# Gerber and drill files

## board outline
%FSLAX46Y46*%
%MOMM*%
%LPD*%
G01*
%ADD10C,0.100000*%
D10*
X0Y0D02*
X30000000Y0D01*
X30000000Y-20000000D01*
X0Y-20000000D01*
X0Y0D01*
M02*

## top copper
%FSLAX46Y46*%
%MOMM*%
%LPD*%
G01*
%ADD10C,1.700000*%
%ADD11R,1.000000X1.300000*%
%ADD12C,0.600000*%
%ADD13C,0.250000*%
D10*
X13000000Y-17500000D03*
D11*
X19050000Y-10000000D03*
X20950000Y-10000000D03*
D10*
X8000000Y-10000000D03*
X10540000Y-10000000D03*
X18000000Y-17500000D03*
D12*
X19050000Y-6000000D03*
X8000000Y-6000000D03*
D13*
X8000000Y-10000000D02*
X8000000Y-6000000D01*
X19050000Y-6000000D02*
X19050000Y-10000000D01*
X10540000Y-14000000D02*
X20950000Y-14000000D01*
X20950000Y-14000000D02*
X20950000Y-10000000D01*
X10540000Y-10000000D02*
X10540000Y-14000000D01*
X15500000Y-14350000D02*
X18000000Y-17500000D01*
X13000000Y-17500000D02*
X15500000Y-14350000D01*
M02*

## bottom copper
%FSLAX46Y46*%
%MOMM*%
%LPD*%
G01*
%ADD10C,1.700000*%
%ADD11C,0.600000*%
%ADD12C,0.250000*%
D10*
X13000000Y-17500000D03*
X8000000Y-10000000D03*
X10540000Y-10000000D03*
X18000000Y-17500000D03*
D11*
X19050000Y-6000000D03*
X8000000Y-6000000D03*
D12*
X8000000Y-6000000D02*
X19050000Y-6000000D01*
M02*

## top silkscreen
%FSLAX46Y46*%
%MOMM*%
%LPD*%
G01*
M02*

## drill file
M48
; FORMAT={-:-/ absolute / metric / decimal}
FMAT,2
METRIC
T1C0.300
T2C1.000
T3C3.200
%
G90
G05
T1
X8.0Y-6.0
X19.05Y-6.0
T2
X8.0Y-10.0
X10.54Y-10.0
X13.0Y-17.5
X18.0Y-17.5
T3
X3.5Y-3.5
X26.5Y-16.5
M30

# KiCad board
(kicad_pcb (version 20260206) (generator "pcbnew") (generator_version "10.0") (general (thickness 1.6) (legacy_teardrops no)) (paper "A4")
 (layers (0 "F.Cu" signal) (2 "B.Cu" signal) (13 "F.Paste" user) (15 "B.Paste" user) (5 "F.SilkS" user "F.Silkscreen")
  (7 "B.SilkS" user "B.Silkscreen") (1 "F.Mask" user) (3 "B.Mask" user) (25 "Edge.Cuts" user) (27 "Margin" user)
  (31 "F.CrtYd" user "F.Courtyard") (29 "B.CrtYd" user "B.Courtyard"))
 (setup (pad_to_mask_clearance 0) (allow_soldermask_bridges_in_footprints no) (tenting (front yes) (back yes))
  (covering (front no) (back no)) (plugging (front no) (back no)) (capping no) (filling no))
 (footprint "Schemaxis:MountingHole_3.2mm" (layer "F.Cu") (at 3.5 3.5)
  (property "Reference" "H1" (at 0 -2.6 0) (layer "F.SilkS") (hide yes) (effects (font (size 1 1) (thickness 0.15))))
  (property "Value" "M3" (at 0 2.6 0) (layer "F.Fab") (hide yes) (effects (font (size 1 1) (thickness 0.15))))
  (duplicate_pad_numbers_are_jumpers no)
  (pad "" np_thru_hole circle (at 0 0) (size 3.2 3.2) (drill 3.2) (layers "*.Cu" "*.Mask")))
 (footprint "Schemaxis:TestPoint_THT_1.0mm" (layer "F.Cu") (at 13 17.5)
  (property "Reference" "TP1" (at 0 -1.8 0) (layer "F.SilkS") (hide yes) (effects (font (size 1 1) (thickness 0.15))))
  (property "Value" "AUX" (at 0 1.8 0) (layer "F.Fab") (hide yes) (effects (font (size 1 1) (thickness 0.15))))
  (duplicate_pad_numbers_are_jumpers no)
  (pad "1" thru_hole circle (at 0 0) (size 1.7 1.7) (drill 1) (layers "*.Cu" "*.Mask") (remove_unused_layers no) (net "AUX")))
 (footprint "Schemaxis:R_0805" (layer "F.Cu") (at 20 10)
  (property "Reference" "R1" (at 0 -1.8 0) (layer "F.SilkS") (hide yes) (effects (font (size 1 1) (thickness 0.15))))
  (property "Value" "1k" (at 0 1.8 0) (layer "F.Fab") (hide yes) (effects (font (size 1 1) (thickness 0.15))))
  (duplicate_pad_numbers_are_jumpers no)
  (pad "1" smd rect (at -0.95 0) (size 1 1.3) (layers "F.Cu" "F.Mask" "F.Paste") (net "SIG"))
  (pad "2" smd rect (at 0.95 0) (size 1 1.3) (layers "F.Cu" "F.Mask" "F.Paste") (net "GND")))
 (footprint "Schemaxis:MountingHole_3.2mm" (layer "F.Cu") (at 26.5 16.5)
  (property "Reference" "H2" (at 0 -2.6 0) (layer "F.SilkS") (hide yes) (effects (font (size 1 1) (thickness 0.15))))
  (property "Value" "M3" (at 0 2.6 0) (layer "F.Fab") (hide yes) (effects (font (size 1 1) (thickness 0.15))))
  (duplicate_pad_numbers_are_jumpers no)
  (pad "" np_thru_hole circle (at 0 0) (size 3.2 3.2) (drill 3.2) (layers "*.Cu" "*.Mask")))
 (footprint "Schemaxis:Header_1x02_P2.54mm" (layer "F.Cu") (at 8 10 90)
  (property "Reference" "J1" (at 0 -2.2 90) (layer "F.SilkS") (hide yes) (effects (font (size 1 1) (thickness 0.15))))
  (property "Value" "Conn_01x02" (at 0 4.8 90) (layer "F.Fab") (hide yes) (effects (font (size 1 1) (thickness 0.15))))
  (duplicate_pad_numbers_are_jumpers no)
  (pad "1" thru_hole circle (at 0 0 90) (size 1.7 1.7) (drill 1) (layers "*.Cu" "*.Mask") (remove_unused_layers no) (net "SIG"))
  (pad "2" thru_hole circle (at 0 2.54 90) (size 1.7 1.7) (drill 1) (layers "*.Cu" "*.Mask") (remove_unused_layers no) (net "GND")))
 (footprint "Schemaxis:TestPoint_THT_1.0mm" (layer "F.Cu") (at 18 17.5)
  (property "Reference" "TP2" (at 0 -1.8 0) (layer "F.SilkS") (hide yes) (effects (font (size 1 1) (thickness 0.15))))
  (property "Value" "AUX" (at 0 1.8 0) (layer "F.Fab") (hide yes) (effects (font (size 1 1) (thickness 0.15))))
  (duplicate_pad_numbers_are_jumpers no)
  (pad "1" thru_hole circle (at 0 0) (size 1.7 1.7) (drill 1) (layers "*.Cu" "*.Mask") (remove_unused_layers no) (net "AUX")))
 (gr_rect (start 0 0) (end 30 20) (stroke (width 0.1) (type default)) (fill no) (layer "Edge.Cuts"))
 (segment (start 8 10) (end 8 6) (width 0.25) (layer "F.Cu") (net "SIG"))
 (segment (start 19.05 6) (end 19.05 10) (width 0.25) (layer "F.Cu") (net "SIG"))
 (via (at 19.05 6) (size 0.6) (drill 0.3) (layers "F.Cu" "B.Cu") (capping no) (covering (front no) (back no))
  (plugging (front no) (back no)) (filling no) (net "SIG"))
 (via (at 8 6) (size 0.6) (drill 0.3) (layers "F.Cu" "B.Cu") (capping no) (covering (front no) (back no)) (plugging (front no) (back no))
  (filling no) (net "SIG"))
 (segment (start 8 6) (end 19.05 6) (width 0.25) (layer "B.Cu") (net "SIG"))
 (segment (start 10.54 14) (end 20.95 14) (width 0.25) (layer "F.Cu") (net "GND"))
 (segment (start 20.95 14) (end 20.95 10) (width 0.25) (layer "F.Cu") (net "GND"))
 (segment (start 10.54 10) (end 10.54 14) (width 0.25) (layer "F.Cu") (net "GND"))
 (segment (start 15.5 14.35) (end 18 17.5) (width 0.25) (layer "F.Cu") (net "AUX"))
 (segment (start 13 17.5) (end 15.5 14.35) (width 0.25) (layer "F.Cu") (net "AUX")))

